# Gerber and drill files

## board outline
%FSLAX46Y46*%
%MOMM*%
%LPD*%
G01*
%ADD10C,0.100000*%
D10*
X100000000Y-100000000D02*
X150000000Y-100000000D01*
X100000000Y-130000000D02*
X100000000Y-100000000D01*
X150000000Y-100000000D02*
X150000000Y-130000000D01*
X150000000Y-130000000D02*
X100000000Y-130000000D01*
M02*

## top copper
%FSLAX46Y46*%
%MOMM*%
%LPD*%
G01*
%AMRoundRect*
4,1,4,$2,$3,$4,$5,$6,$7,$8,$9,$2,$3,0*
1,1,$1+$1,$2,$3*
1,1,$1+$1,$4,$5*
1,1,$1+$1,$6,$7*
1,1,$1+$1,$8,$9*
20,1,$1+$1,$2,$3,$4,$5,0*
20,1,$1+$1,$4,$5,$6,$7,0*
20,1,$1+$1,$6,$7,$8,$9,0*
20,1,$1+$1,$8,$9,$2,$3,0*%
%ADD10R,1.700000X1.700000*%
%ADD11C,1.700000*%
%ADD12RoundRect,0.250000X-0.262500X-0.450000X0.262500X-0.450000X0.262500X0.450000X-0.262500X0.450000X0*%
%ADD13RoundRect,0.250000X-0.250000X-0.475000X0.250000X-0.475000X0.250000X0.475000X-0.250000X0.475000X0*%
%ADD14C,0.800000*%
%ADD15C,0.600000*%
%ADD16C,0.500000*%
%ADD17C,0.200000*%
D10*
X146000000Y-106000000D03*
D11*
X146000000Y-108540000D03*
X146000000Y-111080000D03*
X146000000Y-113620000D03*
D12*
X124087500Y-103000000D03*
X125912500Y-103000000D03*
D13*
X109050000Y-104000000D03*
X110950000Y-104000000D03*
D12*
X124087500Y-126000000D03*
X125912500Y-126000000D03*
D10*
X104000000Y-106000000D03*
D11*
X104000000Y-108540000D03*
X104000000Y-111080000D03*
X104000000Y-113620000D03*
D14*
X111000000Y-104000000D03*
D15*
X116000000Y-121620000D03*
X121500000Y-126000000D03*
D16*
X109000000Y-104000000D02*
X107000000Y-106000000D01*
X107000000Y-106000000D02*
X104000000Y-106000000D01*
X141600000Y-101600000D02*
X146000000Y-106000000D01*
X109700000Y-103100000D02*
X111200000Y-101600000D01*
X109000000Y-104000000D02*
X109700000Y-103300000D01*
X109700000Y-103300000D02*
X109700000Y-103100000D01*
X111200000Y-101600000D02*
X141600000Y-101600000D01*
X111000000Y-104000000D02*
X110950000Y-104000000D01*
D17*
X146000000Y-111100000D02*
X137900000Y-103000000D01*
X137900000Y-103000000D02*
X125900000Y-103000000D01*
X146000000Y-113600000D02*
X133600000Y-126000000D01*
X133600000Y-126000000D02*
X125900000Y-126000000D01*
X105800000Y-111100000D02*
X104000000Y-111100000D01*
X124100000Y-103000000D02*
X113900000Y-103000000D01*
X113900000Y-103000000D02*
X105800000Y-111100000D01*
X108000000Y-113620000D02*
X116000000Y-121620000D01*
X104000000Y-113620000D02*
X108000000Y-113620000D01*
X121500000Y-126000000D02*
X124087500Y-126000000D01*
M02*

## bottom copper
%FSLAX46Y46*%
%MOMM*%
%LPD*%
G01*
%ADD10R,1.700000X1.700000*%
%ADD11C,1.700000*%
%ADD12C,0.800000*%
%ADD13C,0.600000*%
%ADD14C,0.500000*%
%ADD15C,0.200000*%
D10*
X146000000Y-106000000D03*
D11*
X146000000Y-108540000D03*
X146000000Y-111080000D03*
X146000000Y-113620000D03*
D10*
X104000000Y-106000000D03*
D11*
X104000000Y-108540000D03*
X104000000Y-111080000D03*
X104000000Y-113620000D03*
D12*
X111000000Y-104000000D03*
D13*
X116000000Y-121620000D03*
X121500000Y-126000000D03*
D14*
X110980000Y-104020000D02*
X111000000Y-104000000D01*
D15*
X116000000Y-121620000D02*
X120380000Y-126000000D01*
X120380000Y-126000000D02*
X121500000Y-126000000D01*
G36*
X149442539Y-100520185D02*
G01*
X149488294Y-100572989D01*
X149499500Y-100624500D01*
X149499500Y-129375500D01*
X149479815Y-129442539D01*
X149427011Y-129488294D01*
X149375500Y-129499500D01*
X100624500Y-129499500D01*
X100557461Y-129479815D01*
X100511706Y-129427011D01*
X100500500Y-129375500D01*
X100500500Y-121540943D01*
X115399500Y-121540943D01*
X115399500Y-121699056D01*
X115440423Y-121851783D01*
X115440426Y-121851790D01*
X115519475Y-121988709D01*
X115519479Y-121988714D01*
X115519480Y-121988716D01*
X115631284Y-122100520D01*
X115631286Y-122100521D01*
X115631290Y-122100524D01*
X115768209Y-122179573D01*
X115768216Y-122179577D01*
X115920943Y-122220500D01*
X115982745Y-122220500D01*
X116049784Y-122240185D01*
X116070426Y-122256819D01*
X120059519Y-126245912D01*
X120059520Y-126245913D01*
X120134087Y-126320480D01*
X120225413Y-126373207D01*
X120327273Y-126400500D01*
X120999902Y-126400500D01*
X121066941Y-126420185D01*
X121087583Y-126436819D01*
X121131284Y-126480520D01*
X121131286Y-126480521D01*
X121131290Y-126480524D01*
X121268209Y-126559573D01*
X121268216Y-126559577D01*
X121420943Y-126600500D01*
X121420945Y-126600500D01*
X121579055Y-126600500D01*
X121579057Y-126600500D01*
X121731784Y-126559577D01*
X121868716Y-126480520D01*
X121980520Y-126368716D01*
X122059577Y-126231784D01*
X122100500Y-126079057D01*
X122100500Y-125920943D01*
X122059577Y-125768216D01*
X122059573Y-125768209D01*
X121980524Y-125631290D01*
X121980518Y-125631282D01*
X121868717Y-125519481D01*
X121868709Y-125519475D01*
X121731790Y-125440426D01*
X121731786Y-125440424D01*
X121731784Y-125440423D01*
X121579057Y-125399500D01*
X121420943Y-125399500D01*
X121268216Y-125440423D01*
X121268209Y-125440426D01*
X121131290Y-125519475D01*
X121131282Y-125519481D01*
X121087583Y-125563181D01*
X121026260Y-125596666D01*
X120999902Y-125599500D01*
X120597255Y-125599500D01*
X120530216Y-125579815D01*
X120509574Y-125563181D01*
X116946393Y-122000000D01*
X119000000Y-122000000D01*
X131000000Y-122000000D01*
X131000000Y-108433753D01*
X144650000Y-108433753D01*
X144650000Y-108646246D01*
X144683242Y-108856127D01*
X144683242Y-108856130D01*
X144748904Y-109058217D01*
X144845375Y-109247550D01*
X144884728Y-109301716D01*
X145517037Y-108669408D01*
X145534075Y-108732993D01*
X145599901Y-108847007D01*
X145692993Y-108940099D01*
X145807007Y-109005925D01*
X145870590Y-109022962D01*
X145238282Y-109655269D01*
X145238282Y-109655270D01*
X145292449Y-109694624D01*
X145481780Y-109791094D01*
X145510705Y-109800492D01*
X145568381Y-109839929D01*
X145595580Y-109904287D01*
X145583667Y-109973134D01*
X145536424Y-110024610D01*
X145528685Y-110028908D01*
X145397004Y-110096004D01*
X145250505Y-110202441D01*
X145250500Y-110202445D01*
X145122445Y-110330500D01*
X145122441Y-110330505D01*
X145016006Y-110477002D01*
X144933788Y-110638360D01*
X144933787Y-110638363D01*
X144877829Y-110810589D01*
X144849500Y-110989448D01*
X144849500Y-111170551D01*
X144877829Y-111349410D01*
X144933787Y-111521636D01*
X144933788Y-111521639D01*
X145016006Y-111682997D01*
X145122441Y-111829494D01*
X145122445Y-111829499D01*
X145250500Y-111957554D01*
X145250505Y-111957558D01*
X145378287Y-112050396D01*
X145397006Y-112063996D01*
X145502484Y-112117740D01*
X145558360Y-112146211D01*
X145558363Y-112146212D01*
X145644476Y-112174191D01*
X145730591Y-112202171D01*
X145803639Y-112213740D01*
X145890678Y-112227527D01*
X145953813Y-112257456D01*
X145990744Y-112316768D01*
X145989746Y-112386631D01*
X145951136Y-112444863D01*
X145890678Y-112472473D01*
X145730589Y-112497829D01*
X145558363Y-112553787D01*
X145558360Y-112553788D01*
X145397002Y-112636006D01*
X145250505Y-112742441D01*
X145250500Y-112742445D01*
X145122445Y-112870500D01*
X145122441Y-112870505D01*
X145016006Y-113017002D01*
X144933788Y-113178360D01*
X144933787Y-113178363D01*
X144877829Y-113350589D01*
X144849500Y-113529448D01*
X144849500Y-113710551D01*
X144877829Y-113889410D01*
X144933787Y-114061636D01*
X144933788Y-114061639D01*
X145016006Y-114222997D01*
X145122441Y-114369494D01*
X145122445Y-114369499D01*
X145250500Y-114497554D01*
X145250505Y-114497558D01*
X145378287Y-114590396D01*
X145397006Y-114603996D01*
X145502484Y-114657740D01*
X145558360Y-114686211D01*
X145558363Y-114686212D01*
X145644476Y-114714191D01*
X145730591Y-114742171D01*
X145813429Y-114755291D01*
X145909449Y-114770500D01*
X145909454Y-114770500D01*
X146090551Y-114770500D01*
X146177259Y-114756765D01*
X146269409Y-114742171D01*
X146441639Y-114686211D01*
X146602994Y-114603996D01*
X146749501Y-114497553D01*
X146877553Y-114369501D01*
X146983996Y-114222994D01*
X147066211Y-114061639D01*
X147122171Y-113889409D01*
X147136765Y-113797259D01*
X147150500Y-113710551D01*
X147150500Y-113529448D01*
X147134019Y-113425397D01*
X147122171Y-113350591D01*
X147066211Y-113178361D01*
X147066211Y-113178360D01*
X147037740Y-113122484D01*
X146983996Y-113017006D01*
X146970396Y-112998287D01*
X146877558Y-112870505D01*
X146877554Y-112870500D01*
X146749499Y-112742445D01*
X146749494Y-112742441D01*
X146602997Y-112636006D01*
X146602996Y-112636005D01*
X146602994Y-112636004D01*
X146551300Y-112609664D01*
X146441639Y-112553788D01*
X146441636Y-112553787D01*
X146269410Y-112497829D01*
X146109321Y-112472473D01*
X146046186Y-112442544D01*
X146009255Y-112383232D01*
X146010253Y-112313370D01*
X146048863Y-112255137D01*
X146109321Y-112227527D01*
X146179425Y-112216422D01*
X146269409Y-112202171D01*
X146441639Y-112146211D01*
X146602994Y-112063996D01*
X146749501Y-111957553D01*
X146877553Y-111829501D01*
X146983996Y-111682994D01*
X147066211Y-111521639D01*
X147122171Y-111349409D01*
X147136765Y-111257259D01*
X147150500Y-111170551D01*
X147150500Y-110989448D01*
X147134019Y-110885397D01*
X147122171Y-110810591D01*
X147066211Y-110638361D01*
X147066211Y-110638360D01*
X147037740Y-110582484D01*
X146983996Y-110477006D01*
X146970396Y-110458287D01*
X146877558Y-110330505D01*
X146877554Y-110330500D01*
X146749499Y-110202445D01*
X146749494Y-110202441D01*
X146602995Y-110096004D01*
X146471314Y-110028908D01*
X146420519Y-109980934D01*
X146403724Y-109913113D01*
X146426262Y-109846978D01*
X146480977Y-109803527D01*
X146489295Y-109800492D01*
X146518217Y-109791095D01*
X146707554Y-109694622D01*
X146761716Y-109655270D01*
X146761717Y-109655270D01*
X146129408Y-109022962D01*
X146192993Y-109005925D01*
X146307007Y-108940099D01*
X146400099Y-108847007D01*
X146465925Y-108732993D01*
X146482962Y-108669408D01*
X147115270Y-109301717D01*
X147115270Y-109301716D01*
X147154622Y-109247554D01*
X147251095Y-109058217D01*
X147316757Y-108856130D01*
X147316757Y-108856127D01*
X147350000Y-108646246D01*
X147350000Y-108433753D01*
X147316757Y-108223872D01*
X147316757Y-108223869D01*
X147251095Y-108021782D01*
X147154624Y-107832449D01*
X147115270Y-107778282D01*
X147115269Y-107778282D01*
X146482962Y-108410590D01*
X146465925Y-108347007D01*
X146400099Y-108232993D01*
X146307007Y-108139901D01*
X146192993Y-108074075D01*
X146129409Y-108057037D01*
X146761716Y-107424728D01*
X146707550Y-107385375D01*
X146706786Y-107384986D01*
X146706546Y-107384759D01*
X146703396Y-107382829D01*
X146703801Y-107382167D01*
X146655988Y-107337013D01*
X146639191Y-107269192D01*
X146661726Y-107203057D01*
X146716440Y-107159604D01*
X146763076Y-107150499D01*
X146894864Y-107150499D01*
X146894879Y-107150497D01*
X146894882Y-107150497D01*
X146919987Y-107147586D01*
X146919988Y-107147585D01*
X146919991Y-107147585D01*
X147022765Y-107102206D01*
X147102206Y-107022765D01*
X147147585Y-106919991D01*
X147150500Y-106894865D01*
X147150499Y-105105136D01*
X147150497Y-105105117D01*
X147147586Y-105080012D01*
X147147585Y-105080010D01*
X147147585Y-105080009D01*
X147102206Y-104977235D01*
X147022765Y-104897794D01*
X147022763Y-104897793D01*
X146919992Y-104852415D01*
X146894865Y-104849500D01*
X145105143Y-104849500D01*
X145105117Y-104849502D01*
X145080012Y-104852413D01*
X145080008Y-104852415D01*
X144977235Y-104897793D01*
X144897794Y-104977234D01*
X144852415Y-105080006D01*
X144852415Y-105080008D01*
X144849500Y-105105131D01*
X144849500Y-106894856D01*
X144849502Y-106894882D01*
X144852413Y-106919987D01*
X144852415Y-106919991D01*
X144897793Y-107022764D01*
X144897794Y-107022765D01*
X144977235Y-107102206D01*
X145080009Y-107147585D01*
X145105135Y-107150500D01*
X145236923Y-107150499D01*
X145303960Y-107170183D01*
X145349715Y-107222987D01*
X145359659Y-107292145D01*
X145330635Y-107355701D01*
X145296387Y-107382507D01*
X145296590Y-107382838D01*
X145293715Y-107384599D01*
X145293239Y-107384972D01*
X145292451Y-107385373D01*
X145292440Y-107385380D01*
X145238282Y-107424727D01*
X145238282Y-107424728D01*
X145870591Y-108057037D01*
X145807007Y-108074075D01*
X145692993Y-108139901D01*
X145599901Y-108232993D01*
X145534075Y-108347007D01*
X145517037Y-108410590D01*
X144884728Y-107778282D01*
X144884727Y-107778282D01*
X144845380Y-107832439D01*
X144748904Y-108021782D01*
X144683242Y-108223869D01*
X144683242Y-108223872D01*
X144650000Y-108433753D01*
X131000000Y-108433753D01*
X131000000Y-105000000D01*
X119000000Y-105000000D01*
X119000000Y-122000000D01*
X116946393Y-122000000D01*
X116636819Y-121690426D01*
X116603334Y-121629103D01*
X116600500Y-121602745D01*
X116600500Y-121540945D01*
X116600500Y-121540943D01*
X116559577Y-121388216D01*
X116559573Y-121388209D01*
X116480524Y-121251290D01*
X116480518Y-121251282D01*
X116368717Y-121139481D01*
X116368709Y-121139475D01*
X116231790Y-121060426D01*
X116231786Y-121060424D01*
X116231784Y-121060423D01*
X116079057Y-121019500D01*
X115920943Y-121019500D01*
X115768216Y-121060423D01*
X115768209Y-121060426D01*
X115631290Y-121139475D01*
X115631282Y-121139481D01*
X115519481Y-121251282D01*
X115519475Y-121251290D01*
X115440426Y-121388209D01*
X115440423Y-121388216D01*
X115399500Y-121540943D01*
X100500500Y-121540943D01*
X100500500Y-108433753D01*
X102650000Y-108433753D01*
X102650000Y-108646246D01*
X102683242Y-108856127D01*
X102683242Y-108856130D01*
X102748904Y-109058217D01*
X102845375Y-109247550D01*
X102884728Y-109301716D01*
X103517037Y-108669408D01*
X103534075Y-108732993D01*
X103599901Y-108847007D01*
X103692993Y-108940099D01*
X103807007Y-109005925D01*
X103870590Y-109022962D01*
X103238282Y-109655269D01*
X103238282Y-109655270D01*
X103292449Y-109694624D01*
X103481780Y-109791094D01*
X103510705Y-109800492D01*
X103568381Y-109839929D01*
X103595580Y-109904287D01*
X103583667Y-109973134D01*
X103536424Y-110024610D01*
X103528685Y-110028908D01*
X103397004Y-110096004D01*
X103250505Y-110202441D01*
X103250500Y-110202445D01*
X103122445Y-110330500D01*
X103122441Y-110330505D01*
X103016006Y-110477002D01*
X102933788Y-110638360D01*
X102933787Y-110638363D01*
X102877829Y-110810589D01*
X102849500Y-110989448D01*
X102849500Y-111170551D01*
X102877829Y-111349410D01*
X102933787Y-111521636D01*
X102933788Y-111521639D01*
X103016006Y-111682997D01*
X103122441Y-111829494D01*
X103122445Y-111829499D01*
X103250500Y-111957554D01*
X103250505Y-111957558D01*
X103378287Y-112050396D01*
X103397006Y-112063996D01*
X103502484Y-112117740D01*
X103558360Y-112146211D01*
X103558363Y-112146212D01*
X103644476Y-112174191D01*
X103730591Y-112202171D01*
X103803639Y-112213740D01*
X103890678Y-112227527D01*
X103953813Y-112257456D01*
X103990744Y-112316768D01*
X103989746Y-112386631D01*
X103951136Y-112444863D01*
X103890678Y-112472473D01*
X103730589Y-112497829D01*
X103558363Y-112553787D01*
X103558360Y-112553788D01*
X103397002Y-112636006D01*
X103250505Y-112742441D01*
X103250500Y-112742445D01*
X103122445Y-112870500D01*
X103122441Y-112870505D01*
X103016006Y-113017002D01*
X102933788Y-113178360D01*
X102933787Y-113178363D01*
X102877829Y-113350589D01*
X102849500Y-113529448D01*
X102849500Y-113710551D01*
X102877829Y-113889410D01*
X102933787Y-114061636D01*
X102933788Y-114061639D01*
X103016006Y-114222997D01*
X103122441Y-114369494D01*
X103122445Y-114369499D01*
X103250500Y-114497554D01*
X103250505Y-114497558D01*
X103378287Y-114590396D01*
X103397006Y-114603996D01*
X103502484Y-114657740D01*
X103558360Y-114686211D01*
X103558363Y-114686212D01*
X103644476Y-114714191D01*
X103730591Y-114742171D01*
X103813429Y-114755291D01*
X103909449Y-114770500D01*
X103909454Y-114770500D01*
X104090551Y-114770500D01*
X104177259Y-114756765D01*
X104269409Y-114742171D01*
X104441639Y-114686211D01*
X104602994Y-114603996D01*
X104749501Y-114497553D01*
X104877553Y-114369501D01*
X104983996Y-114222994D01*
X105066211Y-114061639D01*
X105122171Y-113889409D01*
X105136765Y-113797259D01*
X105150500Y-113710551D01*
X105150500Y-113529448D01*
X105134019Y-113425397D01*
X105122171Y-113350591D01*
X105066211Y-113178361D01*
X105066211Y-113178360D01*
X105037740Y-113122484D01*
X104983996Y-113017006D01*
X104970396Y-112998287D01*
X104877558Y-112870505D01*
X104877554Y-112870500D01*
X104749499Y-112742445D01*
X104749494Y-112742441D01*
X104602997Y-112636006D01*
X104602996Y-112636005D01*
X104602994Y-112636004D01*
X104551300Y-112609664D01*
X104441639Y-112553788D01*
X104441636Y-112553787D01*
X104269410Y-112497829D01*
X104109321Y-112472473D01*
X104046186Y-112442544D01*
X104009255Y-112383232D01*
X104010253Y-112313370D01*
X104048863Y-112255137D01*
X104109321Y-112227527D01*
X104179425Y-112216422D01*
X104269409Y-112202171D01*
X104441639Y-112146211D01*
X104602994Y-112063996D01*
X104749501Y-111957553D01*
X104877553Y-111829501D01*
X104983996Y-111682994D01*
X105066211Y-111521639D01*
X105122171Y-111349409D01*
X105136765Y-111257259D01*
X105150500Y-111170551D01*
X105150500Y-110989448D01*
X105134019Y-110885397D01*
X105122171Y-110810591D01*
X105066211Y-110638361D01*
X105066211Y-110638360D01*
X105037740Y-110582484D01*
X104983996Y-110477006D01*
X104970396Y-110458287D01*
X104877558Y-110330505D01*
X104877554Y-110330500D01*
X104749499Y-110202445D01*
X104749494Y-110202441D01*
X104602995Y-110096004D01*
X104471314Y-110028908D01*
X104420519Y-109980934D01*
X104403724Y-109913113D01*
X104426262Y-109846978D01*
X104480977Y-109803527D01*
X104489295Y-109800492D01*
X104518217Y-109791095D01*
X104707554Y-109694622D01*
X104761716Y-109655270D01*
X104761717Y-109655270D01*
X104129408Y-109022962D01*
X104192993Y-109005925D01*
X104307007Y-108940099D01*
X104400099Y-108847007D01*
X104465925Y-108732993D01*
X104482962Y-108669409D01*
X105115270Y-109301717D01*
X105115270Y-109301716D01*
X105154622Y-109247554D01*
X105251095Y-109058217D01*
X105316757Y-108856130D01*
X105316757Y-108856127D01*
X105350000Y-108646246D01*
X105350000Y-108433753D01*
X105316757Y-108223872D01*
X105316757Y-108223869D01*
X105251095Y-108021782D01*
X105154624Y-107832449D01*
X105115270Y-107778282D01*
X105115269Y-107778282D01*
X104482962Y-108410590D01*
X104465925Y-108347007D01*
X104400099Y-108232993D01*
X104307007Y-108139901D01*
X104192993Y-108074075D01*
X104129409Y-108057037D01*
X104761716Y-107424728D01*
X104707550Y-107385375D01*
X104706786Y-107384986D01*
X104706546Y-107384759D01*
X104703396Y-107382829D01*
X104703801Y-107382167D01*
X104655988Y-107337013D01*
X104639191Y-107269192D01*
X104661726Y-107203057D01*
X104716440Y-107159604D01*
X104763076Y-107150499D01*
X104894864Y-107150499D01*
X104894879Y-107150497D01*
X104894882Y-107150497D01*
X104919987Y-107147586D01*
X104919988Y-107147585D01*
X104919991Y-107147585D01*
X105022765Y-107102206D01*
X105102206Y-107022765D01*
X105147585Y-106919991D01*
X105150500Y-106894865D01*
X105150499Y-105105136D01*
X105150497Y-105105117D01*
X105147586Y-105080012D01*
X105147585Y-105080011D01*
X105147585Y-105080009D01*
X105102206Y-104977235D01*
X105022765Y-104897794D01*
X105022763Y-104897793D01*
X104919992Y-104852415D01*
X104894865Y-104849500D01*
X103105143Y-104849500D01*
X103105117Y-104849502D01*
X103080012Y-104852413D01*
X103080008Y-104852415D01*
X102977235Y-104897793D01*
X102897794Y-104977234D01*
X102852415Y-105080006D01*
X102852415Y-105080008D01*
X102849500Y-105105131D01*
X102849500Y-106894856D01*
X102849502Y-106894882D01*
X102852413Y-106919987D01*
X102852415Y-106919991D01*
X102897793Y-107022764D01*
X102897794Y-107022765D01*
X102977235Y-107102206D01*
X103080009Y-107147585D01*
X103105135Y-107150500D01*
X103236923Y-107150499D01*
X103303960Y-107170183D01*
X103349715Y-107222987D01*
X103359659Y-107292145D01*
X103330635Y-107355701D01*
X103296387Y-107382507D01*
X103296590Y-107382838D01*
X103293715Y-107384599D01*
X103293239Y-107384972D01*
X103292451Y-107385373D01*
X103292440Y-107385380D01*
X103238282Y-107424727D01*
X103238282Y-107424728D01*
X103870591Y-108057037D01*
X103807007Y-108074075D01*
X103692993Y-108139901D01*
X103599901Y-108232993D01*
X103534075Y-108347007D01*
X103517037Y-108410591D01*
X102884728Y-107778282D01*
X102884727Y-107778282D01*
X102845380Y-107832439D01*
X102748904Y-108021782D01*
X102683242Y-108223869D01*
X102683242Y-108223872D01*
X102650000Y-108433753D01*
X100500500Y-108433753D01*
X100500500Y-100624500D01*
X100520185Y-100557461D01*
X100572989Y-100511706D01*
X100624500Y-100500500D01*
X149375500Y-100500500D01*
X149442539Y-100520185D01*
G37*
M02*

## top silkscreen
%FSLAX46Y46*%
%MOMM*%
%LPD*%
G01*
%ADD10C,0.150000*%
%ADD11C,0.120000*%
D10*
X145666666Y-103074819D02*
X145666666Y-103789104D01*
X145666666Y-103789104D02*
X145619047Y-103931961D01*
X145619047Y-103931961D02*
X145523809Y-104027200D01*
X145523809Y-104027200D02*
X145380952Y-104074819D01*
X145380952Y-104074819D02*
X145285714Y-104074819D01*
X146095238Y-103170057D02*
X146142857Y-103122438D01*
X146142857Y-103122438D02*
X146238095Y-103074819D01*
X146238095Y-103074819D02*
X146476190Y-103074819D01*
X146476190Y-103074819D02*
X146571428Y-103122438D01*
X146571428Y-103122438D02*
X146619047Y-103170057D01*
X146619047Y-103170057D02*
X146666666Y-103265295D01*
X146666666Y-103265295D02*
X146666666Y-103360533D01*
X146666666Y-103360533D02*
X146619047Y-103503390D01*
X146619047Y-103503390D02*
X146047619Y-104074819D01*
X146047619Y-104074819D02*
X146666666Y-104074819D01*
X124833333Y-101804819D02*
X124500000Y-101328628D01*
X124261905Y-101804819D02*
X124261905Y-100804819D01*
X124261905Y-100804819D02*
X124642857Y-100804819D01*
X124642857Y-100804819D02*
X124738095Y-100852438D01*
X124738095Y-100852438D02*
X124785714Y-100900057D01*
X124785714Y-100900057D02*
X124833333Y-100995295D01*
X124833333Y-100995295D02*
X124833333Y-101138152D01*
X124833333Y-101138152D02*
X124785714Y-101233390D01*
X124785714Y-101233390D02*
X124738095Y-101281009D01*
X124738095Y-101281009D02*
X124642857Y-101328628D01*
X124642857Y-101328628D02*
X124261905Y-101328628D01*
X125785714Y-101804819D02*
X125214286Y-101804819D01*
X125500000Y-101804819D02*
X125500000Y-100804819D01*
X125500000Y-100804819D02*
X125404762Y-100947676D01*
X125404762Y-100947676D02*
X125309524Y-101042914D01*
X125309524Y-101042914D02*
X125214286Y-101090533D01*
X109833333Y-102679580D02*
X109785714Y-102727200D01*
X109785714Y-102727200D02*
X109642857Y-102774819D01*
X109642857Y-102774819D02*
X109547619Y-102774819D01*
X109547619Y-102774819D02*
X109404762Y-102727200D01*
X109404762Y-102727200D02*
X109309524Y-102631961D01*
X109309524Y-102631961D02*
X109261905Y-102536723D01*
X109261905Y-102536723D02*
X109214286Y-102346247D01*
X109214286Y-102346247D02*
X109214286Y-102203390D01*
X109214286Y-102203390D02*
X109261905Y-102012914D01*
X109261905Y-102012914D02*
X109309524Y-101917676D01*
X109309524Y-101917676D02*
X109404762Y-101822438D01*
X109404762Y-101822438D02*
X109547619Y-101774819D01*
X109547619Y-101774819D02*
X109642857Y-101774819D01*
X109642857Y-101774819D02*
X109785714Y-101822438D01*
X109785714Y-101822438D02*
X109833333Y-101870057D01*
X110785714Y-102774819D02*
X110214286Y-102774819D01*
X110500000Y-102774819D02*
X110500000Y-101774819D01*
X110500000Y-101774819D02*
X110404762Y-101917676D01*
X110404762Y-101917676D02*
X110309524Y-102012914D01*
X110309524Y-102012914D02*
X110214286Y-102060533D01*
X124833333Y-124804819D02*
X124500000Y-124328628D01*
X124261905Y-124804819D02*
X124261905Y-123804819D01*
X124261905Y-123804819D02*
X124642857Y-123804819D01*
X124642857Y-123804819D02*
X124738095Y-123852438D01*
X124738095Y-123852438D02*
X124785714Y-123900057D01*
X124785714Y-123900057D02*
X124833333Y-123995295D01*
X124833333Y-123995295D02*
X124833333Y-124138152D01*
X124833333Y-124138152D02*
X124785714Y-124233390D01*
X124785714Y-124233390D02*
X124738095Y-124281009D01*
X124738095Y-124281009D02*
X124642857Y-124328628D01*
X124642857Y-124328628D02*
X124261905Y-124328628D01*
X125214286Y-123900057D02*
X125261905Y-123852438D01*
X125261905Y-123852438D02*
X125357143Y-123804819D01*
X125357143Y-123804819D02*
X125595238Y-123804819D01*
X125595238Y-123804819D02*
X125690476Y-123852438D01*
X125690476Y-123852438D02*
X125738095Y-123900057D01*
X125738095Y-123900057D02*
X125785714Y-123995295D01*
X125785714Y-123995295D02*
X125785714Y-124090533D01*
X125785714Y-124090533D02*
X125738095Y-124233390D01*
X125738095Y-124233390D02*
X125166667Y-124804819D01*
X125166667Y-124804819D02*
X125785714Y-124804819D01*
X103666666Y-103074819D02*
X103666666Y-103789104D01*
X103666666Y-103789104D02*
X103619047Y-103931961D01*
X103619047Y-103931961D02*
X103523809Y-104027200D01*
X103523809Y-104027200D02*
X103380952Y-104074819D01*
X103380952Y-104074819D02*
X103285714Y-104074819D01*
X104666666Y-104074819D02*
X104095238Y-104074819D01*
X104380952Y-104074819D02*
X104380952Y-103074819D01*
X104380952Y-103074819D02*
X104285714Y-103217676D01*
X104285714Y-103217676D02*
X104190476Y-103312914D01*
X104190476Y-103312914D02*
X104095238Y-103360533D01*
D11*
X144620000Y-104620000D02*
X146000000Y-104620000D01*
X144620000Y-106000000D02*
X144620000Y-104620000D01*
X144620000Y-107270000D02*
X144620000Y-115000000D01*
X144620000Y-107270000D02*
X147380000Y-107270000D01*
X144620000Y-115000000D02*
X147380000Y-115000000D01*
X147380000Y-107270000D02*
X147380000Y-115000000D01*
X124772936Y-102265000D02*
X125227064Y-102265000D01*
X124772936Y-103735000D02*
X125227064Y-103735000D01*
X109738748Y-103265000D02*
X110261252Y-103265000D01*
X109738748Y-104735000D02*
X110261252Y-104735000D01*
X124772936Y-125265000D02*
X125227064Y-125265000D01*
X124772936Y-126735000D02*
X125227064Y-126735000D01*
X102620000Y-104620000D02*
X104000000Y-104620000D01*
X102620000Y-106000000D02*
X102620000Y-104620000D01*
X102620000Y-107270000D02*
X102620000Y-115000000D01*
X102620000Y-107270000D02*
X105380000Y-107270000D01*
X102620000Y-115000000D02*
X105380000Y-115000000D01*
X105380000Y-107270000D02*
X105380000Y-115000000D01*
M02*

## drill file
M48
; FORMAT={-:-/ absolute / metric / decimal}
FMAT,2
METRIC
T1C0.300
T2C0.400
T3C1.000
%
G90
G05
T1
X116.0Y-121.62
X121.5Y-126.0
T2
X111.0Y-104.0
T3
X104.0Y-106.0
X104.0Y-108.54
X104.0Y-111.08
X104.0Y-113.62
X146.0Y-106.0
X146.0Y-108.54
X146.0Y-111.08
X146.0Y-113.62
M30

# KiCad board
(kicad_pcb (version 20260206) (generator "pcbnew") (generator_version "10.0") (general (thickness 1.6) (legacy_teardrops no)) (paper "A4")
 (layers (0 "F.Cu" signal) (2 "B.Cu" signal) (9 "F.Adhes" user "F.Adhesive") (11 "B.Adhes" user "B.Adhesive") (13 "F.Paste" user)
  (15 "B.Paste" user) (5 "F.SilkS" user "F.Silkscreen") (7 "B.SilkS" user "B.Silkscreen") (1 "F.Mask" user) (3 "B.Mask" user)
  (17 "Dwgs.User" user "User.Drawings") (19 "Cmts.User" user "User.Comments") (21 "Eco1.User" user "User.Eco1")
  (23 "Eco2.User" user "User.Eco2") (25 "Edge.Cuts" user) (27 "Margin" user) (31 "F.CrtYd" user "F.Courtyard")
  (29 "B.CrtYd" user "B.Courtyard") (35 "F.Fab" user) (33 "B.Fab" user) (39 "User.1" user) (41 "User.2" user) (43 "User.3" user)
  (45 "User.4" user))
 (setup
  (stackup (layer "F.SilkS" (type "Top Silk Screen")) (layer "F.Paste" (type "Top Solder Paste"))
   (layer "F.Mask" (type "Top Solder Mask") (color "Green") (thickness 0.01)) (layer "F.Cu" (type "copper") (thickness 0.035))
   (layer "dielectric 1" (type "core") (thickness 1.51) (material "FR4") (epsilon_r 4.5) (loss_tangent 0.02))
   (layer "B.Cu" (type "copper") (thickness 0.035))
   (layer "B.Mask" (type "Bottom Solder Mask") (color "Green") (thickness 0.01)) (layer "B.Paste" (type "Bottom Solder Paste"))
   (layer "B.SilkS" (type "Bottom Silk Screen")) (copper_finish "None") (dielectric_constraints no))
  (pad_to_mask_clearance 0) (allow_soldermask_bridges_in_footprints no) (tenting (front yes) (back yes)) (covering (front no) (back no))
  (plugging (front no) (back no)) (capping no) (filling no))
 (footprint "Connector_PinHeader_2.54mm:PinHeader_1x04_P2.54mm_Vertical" (layer "F.Cu") (at 146 106)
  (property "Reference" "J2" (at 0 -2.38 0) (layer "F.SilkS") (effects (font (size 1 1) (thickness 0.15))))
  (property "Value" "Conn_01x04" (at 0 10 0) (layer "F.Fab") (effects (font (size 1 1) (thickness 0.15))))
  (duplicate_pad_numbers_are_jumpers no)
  (fp_line (start -1.38 -1.38) (end 0 -1.38) (stroke (width 0.12) (type solid)) (layer "F.SilkS"))
  (fp_line (start -1.38 0) (end -1.38 -1.38) (stroke (width 0.12) (type solid)) (layer "F.SilkS"))
  (fp_line (start -1.38 1.27) (end -1.38 9) (stroke (width 0.12) (type solid)) (layer "F.SilkS"))
  (fp_line (start -1.38 1.27) (end 1.38 1.27) (stroke (width 0.12) (type solid)) (layer "F.SilkS"))
  (fp_line (start -1.38 9) (end 1.38 9) (stroke (width 0.12) (type solid)) (layer "F.SilkS"))
  (fp_line (start 1.38 1.27) (end 1.38 9) (stroke (width 0.12) (type solid)) (layer "F.SilkS"))
  (pad "1" thru_hole rect (at 0 0) (size 1.7 1.7) (drill 1) (layers "*.Cu" "*.Mask") (remove_unused_layers no) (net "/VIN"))
  (pad "2" thru_hole circle (at 0 2.54) (size 1.7 1.7) (drill 1) (layers "*.Cu" "*.Mask") (remove_unused_layers no) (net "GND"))
  (pad "3" thru_hole circle (at 0 5.08) (size 1.7 1.7) (drill 1) (layers "*.Cu" "*.Mask") (remove_unused_layers no) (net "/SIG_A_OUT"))
  (pad "4" thru_hole circle (at 0 7.62) (size 1.7 1.7) (drill 1) (layers "*.Cu" "*.Mask") (remove_unused_layers no) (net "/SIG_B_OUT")))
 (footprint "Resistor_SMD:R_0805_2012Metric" (layer "F.Cu") (at 125 103)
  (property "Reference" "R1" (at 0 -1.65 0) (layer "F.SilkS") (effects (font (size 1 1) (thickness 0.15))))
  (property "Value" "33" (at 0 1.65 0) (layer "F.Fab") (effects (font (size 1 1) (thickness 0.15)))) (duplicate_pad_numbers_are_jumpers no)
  (fp_line (start -0.227064 -0.735) (end 0.227064 -0.735) (stroke (width 0.12) (type solid)) (layer "F.SilkS"))
  (fp_line (start -0.227064 0.735) (end 0.227064 0.735) (stroke (width 0.12) (type solid)) (layer "F.SilkS"))
  (pad "1" smd roundrect (at -0.9125 0) (size 1.025 1.4) (layers "F.Cu" "F.Mask" "F.Paste") (roundrect_rratio 0.243902) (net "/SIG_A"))
  (pad "2" smd roundrect (at 0.9125 0) (size 1.025 1.4) (layers "F.Cu" "F.Mask" "F.Paste") (roundrect_rratio 0.243902) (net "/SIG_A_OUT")))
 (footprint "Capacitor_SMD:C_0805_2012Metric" (layer "F.Cu") (at 110 104)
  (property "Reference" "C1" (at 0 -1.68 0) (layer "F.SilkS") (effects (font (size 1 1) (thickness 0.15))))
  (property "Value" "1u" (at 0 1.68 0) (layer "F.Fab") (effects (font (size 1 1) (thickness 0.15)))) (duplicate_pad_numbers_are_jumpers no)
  (fp_line (start -0.261252 -0.735) (end 0.261252 -0.735) (stroke (width 0.12) (type solid)) (layer "F.SilkS"))
  (fp_line (start -0.261252 0.735) (end 0.261252 0.735) (stroke (width 0.12) (type solid)) (layer "F.SilkS"))
  (pad "1" smd roundrect (at -0.95 0) (size 1 1.45) (layers "F.Cu" "F.Mask" "F.Paste") (roundrect_rratio 0.25) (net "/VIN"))
  (pad "2" smd roundrect (at 0.95 0) (size 1 1.45) (layers "F.Cu" "F.Mask" "F.Paste") (roundrect_rratio 0.25) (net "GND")))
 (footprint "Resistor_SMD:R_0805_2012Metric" (layer "F.Cu") (at 125 126)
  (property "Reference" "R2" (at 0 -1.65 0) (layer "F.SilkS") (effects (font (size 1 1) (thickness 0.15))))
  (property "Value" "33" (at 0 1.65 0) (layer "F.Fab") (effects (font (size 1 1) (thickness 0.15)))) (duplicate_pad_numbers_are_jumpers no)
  (fp_line (start -0.227064 -0.735) (end 0.227064 -0.735) (stroke (width 0.12) (type solid)) (layer "F.SilkS"))
  (fp_line (start -0.227064 0.735) (end 0.227064 0.735) (stroke (width 0.12) (type solid)) (layer "F.SilkS"))
  (pad "1" smd roundrect (at -0.9125 0) (size 1.025 1.4) (layers "F.Cu" "F.Mask" "F.Paste") (roundrect_rratio 0.243902) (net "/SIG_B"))
  (pad "2" smd roundrect (at 0.9125 0) (size 1.025 1.4) (layers "F.Cu" "F.Mask" "F.Paste") (roundrect_rratio 0.243902) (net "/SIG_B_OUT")))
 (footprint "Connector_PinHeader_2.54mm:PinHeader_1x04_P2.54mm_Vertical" (layer "F.Cu") (at 104 106)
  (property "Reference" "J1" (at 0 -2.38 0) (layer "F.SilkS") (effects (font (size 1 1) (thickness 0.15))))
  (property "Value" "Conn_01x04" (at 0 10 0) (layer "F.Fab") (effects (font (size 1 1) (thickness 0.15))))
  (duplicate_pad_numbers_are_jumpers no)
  (fp_line (start -1.38 -1.38) (end 0 -1.38) (stroke (width 0.12) (type solid)) (layer "F.SilkS"))
  (fp_line (start -1.38 0) (end -1.38 -1.38) (stroke (width 0.12) (type solid)) (layer "F.SilkS"))
  (fp_line (start -1.38 1.27) (end -1.38 9) (stroke (width 0.12) (type solid)) (layer "F.SilkS"))
  (fp_line (start -1.38 1.27) (end 1.38 1.27) (stroke (width 0.12) (type solid)) (layer "F.SilkS"))
  (fp_line (start -1.38 9) (end 1.38 9) (stroke (width 0.12) (type solid)) (layer "F.SilkS"))
  (fp_line (start 1.38 1.27) (end 1.38 9) (stroke (width 0.12) (type solid)) (layer "F.SilkS"))
  (pad "1" thru_hole rect (at 0 0) (size 1.7 1.7) (drill 1) (layers "*.Cu" "*.Mask") (remove_unused_layers no) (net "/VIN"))
  (pad "2" thru_hole circle (at 0 2.54) (size 1.7 1.7) (drill 1) (layers "*.Cu" "*.Mask") (remove_unused_layers no) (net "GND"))
  (pad "3" thru_hole circle (at 0 5.08) (size 1.7 1.7) (drill 1) (layers "*.Cu" "*.Mask") (remove_unused_layers no) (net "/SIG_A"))
  (pad "4" thru_hole circle (at 0 7.62) (size 1.7 1.7) (drill 1) (layers "*.Cu" "*.Mask") (remove_unused_layers no) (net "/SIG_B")))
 (gr_line (start 100 100) (end 150 100) (stroke (width 0.1) (type default)) (layer "Edge.Cuts"))
 (gr_line (start 100 130) (end 100 100) (stroke (width 0.1) (type default)) (layer "Edge.Cuts"))
 (gr_line (start 150 100) (end 150 130) (stroke (width 0.1) (type default)) (layer "Edge.Cuts"))
 (gr_line (start 150 130) (end 100 130) (stroke (width 0.1) (type default)) (layer "Edge.Cuts"))
 (segment (start 109 104) (end 107 106) (width 0.5) (layer "F.Cu") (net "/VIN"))
 (segment (start 107 106) (end 104 106) (width 0.5) (layer "F.Cu") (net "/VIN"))
 (segment (start 141.6 101.6) (end 146 106) (width 0.5) (layer "F.Cu") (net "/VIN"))
 (segment (start 109.7 103.1) (end 111.2 101.6) (width 0.5) (layer "F.Cu") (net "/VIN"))
 (segment (start 109 104) (end 109.7 103.3) (width 0.5) (layer "F.Cu") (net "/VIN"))
 (segment (start 109.7 103.3) (end 109.7 103.1) (width 0.5) (layer "F.Cu") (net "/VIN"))
 (segment (start 111.2 101.6) (end 141.6 101.6) (width 0.5) (layer "F.Cu") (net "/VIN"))
 (segment (start 111 104) (end 110.95 104) (width 0.5) (layer "F.Cu") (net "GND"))
 (via (at 111 104) (size 0.8) (drill 0.4) (layers "F.Cu" "B.Cu") (capping yes) (filling yes) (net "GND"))
 (segment (start 110.98 104.02) (end 111 104) (width 0.5) (layer "B.Cu") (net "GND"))
 (segment (start 146 111.1) (end 137.9 103) (width 0.2) (layer "F.Cu") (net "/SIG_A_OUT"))
 (segment (start 137.9 103) (end 125.9 103) (width 0.2) (layer "F.Cu") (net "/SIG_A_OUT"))
 (segment (start 146 113.6) (end 133.6 126) (width 0.2) (layer "F.Cu") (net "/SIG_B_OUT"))
 (segment (start 133.6 126) (end 125.9 126) (width 0.2) (layer "F.Cu") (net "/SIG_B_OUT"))
 (segment (start 105.8 111.1) (end 104 111.1) (width 0.2) (layer "F.Cu") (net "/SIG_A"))
 (segment (start 124.1 103) (end 113.9 103) (width 0.2) (layer "F.Cu") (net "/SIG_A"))
 (segment (start 113.9 103) (end 105.8 111.1) (width 0.2) (layer "F.Cu") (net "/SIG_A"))
 (segment (start 108 113.62) (end 116 121.62) (width 0.2) (locked yes) (layer "F.Cu") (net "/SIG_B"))
 (segment (start 104 113.62) (end 108 113.62) (width 0.2) (locked yes) (layer "F.Cu") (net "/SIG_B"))
 (segment (start 121.5 126) (end 124.0875 126) (width 0.2) (locked yes) (layer "F.Cu") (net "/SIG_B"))
 (via (at 116 121.62) (size 0.6) (drill 0.3) (layers "F.Cu" "B.Cu") (locked yes) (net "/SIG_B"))
 (via (at 121.5 126) (size 0.6) (drill 0.3) (layers "F.Cu" "B.Cu") (locked yes) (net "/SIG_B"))
 (segment (start 116 121.62) (end 120.38 126) (width 0.2) (locked yes) (layer "B.Cu") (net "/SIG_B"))
 (segment (start 120.38 126) (end 121.5 126) (width 0.2) (locked yes) (layer "B.Cu") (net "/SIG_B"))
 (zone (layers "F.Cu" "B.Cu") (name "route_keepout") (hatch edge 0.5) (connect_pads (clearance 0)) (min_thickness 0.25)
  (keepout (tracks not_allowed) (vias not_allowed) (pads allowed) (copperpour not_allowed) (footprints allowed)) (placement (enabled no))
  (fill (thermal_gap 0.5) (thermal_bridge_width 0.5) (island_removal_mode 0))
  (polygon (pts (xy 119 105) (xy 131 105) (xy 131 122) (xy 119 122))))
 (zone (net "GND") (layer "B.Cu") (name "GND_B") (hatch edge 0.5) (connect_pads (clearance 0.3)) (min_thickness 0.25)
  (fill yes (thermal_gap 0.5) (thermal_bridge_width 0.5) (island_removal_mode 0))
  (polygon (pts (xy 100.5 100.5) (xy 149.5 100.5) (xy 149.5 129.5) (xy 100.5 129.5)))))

